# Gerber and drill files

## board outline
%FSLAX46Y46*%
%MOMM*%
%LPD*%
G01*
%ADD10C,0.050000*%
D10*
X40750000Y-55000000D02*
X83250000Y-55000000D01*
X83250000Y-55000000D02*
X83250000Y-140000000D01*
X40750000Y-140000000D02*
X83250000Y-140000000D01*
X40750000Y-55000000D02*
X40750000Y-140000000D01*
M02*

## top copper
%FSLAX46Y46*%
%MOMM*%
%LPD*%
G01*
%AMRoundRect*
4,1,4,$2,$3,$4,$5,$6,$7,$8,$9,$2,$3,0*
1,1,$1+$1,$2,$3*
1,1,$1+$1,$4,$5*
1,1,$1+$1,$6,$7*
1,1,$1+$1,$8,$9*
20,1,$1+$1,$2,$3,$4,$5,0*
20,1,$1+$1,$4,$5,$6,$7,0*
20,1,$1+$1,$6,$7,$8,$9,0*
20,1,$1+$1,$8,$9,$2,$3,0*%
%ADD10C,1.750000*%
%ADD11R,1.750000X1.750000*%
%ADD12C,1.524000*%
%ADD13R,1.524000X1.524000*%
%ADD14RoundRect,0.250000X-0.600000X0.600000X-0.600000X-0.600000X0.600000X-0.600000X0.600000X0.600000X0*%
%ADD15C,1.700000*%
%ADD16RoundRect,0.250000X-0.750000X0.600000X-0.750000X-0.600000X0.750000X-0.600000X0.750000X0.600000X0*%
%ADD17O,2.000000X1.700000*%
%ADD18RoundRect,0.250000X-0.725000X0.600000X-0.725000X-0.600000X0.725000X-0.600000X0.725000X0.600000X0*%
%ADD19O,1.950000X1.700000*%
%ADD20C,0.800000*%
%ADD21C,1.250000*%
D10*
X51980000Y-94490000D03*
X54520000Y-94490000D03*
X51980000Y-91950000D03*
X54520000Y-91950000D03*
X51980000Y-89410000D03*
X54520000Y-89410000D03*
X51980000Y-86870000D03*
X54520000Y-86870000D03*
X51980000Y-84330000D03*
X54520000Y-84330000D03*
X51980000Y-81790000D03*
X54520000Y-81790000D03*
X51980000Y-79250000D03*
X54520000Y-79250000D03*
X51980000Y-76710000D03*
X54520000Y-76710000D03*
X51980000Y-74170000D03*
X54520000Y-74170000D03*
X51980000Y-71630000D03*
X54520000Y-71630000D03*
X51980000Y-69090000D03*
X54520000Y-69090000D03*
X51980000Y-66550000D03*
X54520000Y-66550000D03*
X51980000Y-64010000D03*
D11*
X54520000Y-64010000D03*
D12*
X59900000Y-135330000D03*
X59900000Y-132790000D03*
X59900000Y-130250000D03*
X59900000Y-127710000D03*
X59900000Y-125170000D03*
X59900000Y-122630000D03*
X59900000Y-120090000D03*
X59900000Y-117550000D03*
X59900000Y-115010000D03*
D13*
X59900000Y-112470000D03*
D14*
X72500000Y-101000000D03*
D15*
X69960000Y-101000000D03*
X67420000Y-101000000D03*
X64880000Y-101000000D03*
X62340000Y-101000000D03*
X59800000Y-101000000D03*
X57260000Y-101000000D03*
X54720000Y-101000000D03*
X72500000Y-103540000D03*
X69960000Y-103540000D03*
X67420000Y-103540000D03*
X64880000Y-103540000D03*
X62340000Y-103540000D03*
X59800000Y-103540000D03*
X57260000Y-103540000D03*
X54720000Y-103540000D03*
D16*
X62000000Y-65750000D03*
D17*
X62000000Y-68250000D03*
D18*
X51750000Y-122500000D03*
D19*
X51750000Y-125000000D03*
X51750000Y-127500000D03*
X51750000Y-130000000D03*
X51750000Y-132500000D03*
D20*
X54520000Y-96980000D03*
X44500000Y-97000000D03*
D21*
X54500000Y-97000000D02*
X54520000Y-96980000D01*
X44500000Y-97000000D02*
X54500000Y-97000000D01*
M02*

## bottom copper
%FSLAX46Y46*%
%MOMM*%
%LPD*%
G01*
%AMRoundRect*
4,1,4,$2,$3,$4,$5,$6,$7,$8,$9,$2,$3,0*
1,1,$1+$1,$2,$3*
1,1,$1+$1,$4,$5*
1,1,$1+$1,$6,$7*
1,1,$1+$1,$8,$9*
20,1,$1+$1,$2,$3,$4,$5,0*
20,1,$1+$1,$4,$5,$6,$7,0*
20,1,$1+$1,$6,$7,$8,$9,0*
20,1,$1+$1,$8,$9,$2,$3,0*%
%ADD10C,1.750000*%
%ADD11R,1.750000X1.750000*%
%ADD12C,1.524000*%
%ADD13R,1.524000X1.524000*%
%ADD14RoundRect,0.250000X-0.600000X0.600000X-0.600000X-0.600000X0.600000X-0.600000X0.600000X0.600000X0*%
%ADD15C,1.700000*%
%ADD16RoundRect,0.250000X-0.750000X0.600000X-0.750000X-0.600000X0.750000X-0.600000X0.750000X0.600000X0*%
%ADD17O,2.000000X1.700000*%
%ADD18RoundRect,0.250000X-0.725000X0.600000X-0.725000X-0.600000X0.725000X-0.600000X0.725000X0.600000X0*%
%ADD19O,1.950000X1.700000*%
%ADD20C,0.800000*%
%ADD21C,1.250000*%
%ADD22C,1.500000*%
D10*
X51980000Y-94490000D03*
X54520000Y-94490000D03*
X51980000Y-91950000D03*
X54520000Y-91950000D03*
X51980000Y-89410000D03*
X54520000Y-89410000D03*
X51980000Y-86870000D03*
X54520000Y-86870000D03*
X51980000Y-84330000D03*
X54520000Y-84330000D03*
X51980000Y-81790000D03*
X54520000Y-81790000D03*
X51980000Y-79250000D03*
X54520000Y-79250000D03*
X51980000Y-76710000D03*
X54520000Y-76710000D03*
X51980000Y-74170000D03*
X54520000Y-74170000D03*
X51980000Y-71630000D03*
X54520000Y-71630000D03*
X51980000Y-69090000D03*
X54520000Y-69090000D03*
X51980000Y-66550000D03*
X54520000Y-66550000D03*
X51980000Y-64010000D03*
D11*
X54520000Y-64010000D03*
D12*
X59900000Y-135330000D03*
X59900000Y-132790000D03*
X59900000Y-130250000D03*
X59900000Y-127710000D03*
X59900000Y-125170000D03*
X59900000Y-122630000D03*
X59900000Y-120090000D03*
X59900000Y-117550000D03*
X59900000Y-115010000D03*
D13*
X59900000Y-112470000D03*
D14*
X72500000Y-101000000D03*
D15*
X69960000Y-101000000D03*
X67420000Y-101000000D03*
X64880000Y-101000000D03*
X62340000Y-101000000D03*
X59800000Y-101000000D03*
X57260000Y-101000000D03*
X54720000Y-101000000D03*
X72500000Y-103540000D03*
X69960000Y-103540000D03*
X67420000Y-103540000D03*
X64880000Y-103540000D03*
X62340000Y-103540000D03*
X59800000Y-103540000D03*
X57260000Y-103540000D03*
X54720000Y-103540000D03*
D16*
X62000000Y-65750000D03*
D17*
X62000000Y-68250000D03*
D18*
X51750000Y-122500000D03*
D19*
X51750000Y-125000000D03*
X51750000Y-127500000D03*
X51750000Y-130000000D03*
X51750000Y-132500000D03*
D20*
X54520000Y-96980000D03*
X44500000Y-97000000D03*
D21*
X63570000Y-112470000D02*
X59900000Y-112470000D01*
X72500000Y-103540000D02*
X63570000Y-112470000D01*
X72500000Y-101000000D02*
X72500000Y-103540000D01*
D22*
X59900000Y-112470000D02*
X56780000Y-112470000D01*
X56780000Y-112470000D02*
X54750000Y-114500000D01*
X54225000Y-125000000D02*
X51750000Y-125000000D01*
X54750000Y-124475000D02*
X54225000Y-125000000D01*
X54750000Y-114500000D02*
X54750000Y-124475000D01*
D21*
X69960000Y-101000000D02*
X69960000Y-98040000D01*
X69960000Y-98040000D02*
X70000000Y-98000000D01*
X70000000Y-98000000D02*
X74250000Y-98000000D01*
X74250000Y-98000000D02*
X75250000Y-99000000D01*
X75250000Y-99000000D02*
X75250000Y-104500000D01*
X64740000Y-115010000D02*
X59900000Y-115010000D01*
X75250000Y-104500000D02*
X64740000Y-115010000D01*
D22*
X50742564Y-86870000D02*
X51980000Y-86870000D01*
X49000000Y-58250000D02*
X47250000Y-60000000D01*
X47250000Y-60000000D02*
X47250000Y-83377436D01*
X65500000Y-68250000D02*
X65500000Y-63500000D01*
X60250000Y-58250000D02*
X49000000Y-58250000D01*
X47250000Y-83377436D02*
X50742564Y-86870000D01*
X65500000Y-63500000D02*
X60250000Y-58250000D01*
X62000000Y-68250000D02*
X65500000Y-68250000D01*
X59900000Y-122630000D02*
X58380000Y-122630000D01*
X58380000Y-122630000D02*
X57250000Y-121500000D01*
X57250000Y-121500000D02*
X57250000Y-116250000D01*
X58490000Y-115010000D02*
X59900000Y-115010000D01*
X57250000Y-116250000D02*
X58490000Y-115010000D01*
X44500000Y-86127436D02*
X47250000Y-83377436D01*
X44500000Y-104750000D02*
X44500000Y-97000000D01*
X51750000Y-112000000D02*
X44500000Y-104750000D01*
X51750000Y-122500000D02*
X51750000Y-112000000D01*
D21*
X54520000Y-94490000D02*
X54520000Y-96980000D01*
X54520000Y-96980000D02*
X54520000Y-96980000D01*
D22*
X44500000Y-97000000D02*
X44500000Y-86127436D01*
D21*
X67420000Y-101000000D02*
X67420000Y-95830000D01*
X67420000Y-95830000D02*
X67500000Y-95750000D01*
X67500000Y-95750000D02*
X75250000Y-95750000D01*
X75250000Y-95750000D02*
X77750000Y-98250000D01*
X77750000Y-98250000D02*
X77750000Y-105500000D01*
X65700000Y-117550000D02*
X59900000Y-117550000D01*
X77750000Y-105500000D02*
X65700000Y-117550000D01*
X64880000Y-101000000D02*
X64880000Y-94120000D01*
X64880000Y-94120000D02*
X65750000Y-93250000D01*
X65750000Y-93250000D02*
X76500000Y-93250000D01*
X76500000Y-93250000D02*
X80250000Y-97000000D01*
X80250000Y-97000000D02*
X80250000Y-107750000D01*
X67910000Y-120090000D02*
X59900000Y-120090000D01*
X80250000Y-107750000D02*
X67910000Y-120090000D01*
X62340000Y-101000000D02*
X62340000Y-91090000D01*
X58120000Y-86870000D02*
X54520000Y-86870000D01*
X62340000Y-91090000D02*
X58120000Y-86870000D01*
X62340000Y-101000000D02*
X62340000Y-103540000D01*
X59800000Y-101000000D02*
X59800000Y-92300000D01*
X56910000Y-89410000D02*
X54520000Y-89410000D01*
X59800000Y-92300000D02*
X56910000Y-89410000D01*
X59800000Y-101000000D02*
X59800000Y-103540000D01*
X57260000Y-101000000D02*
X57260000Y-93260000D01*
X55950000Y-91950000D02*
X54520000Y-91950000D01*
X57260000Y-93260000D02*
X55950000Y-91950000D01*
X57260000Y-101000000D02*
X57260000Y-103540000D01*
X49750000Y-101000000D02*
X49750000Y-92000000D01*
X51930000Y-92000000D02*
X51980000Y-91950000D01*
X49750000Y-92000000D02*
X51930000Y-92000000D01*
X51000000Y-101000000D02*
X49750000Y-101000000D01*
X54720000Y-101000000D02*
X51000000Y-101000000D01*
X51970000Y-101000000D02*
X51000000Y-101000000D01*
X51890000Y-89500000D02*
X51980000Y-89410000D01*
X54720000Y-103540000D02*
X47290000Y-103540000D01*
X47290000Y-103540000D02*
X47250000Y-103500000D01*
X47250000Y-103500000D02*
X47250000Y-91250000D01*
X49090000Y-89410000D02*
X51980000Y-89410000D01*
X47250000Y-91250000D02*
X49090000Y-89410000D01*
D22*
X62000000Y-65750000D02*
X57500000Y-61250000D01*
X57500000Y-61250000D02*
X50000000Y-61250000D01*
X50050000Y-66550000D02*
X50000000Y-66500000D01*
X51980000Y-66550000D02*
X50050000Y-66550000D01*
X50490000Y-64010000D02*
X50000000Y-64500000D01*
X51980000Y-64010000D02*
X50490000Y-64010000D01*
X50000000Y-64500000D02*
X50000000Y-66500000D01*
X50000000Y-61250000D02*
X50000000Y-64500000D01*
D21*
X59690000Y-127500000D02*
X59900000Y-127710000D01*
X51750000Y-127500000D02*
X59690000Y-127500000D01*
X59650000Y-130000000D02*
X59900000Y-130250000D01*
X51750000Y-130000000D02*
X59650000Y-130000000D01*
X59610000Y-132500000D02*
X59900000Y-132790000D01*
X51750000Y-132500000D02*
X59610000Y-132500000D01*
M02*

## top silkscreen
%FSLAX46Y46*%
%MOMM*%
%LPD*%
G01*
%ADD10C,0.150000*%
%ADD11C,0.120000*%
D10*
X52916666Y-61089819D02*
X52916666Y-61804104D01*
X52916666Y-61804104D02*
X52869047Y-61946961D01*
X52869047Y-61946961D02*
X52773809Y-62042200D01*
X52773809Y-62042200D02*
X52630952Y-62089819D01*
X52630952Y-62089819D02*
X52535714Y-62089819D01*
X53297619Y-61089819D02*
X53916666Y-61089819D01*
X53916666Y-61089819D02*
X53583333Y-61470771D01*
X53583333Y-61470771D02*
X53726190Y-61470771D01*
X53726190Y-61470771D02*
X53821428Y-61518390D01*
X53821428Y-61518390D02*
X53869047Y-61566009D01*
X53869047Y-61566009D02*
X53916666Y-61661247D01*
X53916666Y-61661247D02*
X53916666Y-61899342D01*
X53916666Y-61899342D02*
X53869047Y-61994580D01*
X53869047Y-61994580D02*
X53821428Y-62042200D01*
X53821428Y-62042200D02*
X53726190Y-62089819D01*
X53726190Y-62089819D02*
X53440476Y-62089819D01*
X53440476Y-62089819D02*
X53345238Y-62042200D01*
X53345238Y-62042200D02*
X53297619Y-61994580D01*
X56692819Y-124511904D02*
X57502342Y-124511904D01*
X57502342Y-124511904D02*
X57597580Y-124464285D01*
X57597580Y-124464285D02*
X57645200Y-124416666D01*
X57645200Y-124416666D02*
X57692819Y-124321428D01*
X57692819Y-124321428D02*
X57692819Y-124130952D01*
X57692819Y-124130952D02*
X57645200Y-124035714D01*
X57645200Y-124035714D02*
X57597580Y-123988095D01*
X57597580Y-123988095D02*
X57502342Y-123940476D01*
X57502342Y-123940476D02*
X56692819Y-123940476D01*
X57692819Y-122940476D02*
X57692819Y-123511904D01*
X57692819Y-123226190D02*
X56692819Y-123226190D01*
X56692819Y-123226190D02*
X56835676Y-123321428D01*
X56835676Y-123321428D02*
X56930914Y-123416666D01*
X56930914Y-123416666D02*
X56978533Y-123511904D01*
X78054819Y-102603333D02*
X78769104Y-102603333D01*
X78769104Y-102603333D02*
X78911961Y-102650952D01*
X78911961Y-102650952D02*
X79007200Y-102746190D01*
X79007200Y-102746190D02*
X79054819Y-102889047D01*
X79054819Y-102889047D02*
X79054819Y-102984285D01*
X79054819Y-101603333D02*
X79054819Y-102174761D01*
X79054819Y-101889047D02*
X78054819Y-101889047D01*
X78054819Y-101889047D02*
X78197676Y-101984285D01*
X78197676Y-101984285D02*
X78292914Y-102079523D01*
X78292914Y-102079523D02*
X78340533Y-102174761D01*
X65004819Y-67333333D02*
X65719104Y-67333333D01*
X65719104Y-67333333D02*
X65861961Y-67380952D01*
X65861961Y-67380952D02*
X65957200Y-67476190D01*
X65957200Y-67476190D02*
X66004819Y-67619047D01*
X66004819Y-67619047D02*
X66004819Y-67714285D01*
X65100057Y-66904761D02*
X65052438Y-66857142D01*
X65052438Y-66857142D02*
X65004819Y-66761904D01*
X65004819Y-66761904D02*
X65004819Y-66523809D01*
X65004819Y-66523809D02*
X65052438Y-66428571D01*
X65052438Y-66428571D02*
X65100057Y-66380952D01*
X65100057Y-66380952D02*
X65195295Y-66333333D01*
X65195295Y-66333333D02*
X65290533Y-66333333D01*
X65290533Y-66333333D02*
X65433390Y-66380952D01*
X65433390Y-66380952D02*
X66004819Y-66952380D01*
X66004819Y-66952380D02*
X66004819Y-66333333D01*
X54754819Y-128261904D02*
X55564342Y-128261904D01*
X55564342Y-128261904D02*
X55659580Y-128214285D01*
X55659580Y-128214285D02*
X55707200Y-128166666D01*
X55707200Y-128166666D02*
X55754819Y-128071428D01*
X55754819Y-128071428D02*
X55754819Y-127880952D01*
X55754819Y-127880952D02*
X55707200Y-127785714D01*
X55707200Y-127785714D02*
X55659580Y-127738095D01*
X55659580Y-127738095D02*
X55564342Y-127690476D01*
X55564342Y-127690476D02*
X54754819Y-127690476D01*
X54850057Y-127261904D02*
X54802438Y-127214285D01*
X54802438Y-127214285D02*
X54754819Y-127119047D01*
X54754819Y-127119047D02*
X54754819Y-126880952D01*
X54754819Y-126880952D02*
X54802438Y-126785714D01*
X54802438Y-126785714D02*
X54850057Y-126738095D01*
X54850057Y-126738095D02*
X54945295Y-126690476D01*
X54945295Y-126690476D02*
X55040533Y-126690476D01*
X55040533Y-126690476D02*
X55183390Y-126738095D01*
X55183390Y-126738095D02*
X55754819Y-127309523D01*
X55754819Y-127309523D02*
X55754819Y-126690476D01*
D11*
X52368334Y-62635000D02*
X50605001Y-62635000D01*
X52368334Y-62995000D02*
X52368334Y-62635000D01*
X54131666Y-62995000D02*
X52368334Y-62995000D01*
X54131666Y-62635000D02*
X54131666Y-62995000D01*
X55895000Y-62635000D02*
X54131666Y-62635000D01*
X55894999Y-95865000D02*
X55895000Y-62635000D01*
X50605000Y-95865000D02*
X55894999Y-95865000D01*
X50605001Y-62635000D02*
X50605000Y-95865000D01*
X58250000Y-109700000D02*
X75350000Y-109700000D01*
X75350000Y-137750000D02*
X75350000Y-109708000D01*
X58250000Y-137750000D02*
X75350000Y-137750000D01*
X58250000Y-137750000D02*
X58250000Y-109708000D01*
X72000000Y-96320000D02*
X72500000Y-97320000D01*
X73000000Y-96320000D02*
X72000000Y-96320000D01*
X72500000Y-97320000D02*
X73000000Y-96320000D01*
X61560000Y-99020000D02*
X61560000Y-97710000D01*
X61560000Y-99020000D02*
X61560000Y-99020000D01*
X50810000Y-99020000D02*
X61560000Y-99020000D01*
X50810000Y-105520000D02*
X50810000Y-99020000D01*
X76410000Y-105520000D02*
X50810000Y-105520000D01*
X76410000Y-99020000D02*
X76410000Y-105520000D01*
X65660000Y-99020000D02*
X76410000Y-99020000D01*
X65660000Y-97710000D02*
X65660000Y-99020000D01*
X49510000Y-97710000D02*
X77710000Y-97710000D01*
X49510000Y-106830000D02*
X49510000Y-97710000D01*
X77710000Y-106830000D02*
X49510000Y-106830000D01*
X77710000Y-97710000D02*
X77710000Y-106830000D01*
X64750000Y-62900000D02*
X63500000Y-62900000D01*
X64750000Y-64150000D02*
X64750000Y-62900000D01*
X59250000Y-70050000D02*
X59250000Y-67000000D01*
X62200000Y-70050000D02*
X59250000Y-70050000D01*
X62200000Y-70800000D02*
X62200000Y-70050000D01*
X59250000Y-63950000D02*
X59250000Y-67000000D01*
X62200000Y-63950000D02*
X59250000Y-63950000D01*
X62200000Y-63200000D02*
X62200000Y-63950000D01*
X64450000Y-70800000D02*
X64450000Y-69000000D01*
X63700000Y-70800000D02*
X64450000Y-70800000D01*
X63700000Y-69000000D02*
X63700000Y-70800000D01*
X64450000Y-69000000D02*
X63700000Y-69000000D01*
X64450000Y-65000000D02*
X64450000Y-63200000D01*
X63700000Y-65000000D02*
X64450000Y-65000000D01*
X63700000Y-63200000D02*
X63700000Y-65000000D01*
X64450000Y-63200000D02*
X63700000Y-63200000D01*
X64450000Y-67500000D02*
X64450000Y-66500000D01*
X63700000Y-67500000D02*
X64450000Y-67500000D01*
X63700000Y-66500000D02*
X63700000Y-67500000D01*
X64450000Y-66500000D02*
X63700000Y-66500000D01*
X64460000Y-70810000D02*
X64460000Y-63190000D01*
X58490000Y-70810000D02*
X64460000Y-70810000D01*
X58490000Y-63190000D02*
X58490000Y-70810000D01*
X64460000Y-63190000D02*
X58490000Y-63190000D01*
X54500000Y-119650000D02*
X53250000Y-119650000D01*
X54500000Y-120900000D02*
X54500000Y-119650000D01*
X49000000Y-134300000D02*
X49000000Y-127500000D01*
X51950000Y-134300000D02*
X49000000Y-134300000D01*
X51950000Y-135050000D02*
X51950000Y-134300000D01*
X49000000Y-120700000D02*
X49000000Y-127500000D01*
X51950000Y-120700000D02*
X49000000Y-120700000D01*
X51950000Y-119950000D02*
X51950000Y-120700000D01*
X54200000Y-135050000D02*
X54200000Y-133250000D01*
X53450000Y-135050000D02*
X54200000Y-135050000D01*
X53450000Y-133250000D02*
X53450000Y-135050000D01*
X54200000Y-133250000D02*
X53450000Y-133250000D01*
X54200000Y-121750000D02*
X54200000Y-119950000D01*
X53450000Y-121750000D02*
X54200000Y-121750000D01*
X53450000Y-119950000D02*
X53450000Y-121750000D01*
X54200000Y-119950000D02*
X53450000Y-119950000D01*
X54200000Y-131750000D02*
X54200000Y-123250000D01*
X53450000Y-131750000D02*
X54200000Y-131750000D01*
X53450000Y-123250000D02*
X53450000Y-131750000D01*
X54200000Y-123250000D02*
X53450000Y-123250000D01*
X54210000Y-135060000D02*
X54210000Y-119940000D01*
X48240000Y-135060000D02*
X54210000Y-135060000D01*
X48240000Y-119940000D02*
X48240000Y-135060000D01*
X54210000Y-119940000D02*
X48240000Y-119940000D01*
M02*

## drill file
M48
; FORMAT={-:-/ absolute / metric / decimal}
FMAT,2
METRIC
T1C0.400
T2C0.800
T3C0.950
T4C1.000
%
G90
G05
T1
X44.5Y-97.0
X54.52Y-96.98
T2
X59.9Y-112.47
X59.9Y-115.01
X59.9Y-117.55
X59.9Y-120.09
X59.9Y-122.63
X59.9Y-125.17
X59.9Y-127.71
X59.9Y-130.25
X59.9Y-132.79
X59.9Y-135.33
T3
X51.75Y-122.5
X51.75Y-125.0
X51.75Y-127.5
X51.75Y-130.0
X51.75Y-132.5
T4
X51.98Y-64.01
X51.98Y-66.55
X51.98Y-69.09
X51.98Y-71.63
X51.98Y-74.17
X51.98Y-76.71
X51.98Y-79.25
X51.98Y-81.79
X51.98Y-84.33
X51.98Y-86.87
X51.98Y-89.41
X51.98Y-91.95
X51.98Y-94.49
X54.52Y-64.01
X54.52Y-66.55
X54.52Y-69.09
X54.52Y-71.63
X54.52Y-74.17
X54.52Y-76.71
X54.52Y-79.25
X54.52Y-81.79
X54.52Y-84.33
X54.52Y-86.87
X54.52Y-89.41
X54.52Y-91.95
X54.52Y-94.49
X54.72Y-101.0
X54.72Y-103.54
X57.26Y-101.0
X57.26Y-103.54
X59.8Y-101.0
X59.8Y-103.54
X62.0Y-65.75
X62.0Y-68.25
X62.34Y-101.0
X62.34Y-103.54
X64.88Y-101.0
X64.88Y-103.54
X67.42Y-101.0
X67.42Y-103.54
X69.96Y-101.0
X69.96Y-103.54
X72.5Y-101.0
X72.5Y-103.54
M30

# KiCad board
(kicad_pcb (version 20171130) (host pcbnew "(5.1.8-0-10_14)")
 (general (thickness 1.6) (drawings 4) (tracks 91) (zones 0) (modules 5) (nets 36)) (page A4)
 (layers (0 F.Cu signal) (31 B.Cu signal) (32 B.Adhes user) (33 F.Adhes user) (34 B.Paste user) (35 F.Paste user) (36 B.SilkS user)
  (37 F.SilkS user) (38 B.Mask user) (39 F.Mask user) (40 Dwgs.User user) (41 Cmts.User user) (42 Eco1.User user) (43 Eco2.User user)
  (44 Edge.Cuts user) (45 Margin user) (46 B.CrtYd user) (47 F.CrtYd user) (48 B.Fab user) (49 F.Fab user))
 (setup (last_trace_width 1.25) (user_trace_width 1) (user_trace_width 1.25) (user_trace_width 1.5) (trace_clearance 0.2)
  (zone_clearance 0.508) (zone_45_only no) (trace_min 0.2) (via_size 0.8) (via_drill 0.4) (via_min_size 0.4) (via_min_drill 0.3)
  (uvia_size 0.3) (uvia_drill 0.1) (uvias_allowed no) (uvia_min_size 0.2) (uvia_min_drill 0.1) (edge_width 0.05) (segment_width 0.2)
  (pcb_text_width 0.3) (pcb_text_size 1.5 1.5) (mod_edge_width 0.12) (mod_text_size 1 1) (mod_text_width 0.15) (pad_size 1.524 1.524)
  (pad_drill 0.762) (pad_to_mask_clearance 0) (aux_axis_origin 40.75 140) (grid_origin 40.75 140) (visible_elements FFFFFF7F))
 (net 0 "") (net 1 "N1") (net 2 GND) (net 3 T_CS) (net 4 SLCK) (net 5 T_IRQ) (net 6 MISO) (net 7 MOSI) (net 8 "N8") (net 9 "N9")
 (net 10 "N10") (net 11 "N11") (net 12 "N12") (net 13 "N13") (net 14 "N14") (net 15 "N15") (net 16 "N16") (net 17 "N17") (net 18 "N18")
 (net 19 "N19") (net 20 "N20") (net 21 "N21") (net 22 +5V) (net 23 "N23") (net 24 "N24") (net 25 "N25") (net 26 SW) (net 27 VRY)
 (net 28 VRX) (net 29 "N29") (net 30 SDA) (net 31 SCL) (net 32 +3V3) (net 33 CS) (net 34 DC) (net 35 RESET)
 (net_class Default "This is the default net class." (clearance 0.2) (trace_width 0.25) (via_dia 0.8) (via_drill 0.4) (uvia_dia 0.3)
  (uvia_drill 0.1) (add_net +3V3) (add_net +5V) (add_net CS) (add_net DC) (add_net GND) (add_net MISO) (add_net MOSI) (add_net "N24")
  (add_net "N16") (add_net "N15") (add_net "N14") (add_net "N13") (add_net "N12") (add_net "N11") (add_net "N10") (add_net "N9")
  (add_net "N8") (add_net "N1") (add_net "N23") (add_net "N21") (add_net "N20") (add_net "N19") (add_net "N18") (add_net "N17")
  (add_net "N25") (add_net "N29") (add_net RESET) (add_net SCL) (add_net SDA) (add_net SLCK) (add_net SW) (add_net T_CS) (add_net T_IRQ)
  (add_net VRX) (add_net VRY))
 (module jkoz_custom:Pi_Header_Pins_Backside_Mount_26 (layer F.Cu) (at 53.25 79.25 270)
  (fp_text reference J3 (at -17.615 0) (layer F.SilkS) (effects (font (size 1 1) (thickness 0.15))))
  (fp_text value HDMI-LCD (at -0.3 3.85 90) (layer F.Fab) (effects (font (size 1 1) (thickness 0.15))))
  (fp_line (start -16.615 0.881666) (end -16.615 2.644999) (layer F.SilkS) (width 0.12))
  (fp_line (start -16.255 0.881666) (end -16.615 0.881666) (layer F.SilkS) (width 0.12))
  (fp_line (start -16.255 -0.881666) (end -16.255 0.881666) (layer F.SilkS) (width 0.12))
  (fp_line (start -16.615 -0.881666) (end -16.255 -0.881666) (layer F.SilkS) (width 0.12))
  (fp_line (start -16.615 -2.645) (end -16.615 -0.881666) (layer F.SilkS) (width 0.12))
  (fp_line (start 16.615 -2.644999) (end -16.615 -2.645) (layer F.SilkS) (width 0.12))
  (fp_line (start 16.615 2.645) (end 16.615 -2.644999) (layer F.SilkS) (width 0.12))
  (fp_line (start -16.615 2.644999) (end 16.615 2.645) (layer F.SilkS) (width 0.12))
  (pad 26 thru_hole circle (at 15.24 1.27 270) (size 1.75 1.75) (drill 1) (layers *.Cu *.Mask) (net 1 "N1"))
  (pad 25 thru_hole circle (at 15.24 -1.27 270) (size 1.75 1.75) (drill 1) (layers *.Cu *.Mask) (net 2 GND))
  (pad 24 thru_hole circle (at 12.7 1.27 270) (size 1.75 1.75) (drill 1) (layers *.Cu *.Mask) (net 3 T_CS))
  (pad 23 thru_hole circle (at 12.7 -1.27 270) (size 1.75 1.75) (drill 1) (layers *.Cu *.Mask) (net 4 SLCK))
  (pad 22 thru_hole circle (at 10.16 1.27 270) (size 1.75 1.75) (drill 1) (layers *.Cu *.Mask) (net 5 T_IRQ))
  (pad 21 thru_hole circle (at 10.16 -1.27 270) (size 1.75 1.75) (drill 1) (layers *.Cu *.Mask) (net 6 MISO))
  (pad 20 thru_hole circle (at 7.62 1.27 270) (size 1.75 1.75) (drill 1) (layers *.Cu *.Mask) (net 2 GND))
  (pad 19 thru_hole circle (at 7.62 -1.27 270) (size 1.75 1.75) (drill 1) (layers *.Cu *.Mask) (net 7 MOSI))
  (pad 18 thru_hole circle (at 5.08 1.27 270) (size 1.75 1.75) (drill 1) (layers *.Cu *.Mask) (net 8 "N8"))
  (pad 17 thru_hole circle (at 5.08 -1.27 270) (size 1.75 1.75) (drill 1) (layers *.Cu *.Mask) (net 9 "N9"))
  (pad 16 thru_hole circle (at 2.54 1.27 270) (size 1.75 1.75) (drill 1) (layers *.Cu *.Mask) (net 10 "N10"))
  (pad 15 thru_hole circle (at 2.54 -1.27 270) (size 1.75 1.75) (drill 1) (layers *.Cu *.Mask) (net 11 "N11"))
  (pad 14 thru_hole circle (at 0 1.27 270) (size 1.75 1.75) (drill 1) (layers *.Cu *.Mask) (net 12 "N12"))
  (pad 13 thru_hole circle (at 0 -1.27 270) (size 1.75 1.75) (drill 1) (layers *.Cu *.Mask) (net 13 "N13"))
  (pad 12 thru_hole circle (at -2.54 1.27 270) (size 1.75 1.75) (drill 1) (layers *.Cu *.Mask) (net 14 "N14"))
  (pad 11 thru_hole circle (at -2.54 -1.27 270) (size 1.75 1.75) (drill 1) (layers *.Cu *.Mask) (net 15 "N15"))
  (pad 10 thru_hole circle (at -5.08 1.27 270) (size 1.75 1.75) (drill 1) (layers *.Cu *.Mask) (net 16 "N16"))
  (pad 9 thru_hole circle (at -5.08 -1.27 270) (size 1.75 1.75) (drill 1) (layers *.Cu *.Mask) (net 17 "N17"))
  (pad 8 thru_hole circle (at -7.62 1.27 270) (size 1.75 1.75) (drill 1) (layers *.Cu *.Mask) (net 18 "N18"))
  (pad 7 thru_hole circle (at -7.62 -1.27 270) (size 1.75 1.75) (drill 1) (layers *.Cu *.Mask) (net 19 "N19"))
  (pad 6 thru_hole circle (at -10.16 1.27 270) (size 1.75 1.75) (drill 1) (layers *.Cu *.Mask) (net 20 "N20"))
  (pad 5 thru_hole circle (at -10.16 -1.27 270) (size 1.75 1.75) (drill 1) (layers *.Cu *.Mask) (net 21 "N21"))
  (pad 4 thru_hole circle (at -12.7 1.27 270) (size 1.75 1.75) (drill 1) (layers *.Cu *.Mask) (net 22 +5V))
  (pad 3 thru_hole circle (at -12.7 -1.27 270) (size 1.75 1.75) (drill 1) (layers *.Cu *.Mask) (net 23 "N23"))
  (pad 2 thru_hole circle (at -15.24 1.27 270) (size 1.75 1.75) (drill 1) (layers *.Cu *.Mask) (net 22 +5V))
  (pad 1 thru_hole rect (at -15.24 -1.27 270) (size 1.75 1.75) (drill 1) (layers *.Cu *.Mask) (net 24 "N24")))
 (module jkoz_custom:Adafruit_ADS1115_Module (layer F.Cu) (at 59.5 123.75 270)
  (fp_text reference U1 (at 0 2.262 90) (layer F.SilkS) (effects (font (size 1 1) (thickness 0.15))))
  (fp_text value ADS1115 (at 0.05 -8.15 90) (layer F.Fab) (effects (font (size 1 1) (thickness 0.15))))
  (fp_line (start -14.05 1.25) (end -14.05 -15.85) (layer F.SilkS) (width 0.12))
  (fp_line (start 14 -15.85) (end -14.042 -15.85) (layer F.SilkS) (width 0.12))
  (fp_line (start 14 1.25) (end 14 -15.85) (layer F.SilkS) (width 0.12))
  (fp_line (start 14 1.25) (end -14.042 1.25) (layer F.SilkS) (width 0.12))
  (pad 10 thru_hole circle (at 11.58 -0.4 270) (size 1.524 1.524) (drill 0.8) (layers *.Cu *.Mask) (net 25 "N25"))
  (pad 9 thru_hole circle (at 9.04 -0.4 270) (size 1.524 1.524) (drill 0.8) (layers *.Cu *.Mask) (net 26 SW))
  (pad 8 thru_hole circle (at 6.5 -0.4 270) (size 1.524 1.524) (drill 0.8) (layers *.Cu *.Mask) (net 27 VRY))
  (pad 7 thru_hole circle (at 3.96 -0.4 270) (size 1.524 1.524) (drill 0.8) (layers *.Cu *.Mask) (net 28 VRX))
  (pad 6 thru_hole circle (at 1.42 -0.4 270) (size 1.524 1.524) (drill 0.8) (layers *.Cu *.Mask) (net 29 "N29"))
  (pad 5 thru_hole circle (at -1.12 -0.4 270) (size 1.524 1.524) (drill 0.8) (layers *.Cu *.Mask) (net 2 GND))
  (pad 4 thru_hole circle (at -3.66 -0.4 270) (size 1.524 1.524) (drill 0.8) (layers *.Cu *.Mask) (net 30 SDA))
  (pad 3 thru_hole circle (at -6.2 -0.4 270) (size 1.524 1.524) (drill 0.8) (layers *.Cu *.Mask) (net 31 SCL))
  (pad 2 thru_hole circle (at -8.74 -0.4 270) (size 1.524 1.524) (drill 0.8) (layers *.Cu *.Mask) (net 2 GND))
  (pad 1 thru_hole rect (at -11.28 -0.4 270) (size 1.524 1.524) (drill 0.8) (layers *.Cu *.Mask) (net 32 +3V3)))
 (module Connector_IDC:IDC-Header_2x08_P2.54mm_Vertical (layer F.Cu) (at 72.5 101 270)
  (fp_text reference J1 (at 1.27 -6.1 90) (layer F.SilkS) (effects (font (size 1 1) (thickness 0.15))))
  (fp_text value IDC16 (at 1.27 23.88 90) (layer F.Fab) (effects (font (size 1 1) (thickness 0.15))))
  (fp_line (start -4.68 0.5) (end -3.68 0) (layer F.SilkS) (width 0.12))
  (fp_line (start -4.68 -0.5) (end -4.68 0.5) (layer F.SilkS) (width 0.12))
  (fp_line (start -3.68 0) (end -4.68 -0.5) (layer F.SilkS) (width 0.12))
  (fp_line (start -1.98 10.94) (end -3.29 10.94) (layer F.SilkS) (width 0.12))
  (fp_line (start -1.98 10.94) (end -1.98 10.94) (layer F.SilkS) (width 0.12))
  (fp_line (start -1.98 21.69) (end -1.98 10.94) (layer F.SilkS) (width 0.12))
  (fp_line (start 4.52 21.69) (end -1.98 21.69) (layer F.SilkS) (width 0.12))
  (fp_line (start 4.52 -3.91) (end 4.52 21.69) (layer F.SilkS) (width 0.12))
  (fp_line (start -1.98 -3.91) (end 4.52 -3.91) (layer F.SilkS) (width 0.12))
  (fp_line (start -1.98 6.84) (end -1.98 -3.91) (layer F.SilkS) (width 0.12))
  (fp_line (start -3.29 6.84) (end -1.98 6.84) (layer F.SilkS) (width 0.12))
  (fp_line (start -3.29 22.99) (end -3.29 -5.21) (layer F.SilkS) (width 0.12))
  (fp_line (start 5.83 22.99) (end -3.29 22.99) (layer F.SilkS) (width 0.12))
  (fp_line (start 5.83 -5.21) (end 5.83 22.99) (layer F.SilkS) (width 0.12))
  (fp_line (start -3.29 -5.21) (end 5.83 -5.21) (layer F.SilkS) (width 0.12))
  (pad 1 thru_hole roundrect (at 0 0 270) (size 1.7 1.7) (drill 1) (layers *.Cu *.Mask) (roundrect_rratio 0.1470588235294118) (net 32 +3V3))
  (pad 3 thru_hole circle (at 0 2.54 270) (size 1.7 1.7) (drill 1) (layers *.Cu *.Mask) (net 2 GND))
  (pad 5 thru_hole circle (at 0 5.08 270) (size 1.7 1.7) (drill 1) (layers *.Cu *.Mask) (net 31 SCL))
  (pad 7 thru_hole circle (at 0 7.62 270) (size 1.7 1.7) (drill 1) (layers *.Cu *.Mask) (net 30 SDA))
  (pad 9 thru_hole circle (at 0 10.16 270) (size 1.7 1.7) (drill 1) (layers *.Cu *.Mask) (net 7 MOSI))
  (pad 11 thru_hole circle (at 0 12.7 270) (size 1.7 1.7) (drill 1) (layers *.Cu *.Mask) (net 6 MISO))
  (pad 13 thru_hole circle (at 0 15.24 270) (size 1.7 1.7) (drill 1) (layers *.Cu *.Mask) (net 4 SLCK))
  (pad 15 thru_hole circle (at 0 17.78 270) (size 1.7 1.7) (drill 1) (layers *.Cu *.Mask) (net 3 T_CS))
  (pad 2 thru_hole circle (at 2.54 0 270) (size 1.7 1.7) (drill 1) (layers *.Cu *.Mask) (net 32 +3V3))
  (pad 4 thru_hole circle (at 2.54 2.54 270) (size 1.7 1.7) (drill 1) (layers *.Cu *.Mask) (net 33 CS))
  (pad 6 thru_hole circle (at 2.54 5.08 270) (size 1.7 1.7) (drill 1) (layers *.Cu *.Mask) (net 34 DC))
  (pad 8 thru_hole circle (at 2.54 7.62 270) (size 1.7 1.7) (drill 1) (layers *.Cu *.Mask) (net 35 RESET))
  (pad 10 thru_hole circle (at 2.54 10.16 270) (size 1.7 1.7) (drill 1) (layers *.Cu *.Mask) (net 7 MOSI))
  (pad 12 thru_hole circle (at 2.54 12.7 270) (size 1.7 1.7) (drill 1) (layers *.Cu *.Mask) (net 6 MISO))
  (pad 14 thru_hole circle (at 2.54 15.24 270) (size 1.7 1.7) (drill 1) (layers *.Cu *.Mask) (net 4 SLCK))
  (pad 16 thru_hole circle (at 2.54 17.78 270) (size 1.7 1.7) (drill 1) (layers *.Cu *.Mask) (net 5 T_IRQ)))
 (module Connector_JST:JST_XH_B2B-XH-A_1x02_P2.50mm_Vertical (layer F.Cu) (at 62 65.75 270)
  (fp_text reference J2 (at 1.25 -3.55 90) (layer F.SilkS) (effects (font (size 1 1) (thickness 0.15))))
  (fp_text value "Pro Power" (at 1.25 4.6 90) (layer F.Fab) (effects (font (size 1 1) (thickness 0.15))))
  (fp_line (start -2.85 -2.75) (end -2.85 -1.5) (layer F.SilkS) (width 0.12))
  (fp_line (start -1.6 -2.75) (end -2.85 -2.75) (layer F.SilkS) (width 0.12))
  (fp_line (start 4.3 2.75) (end 1.25 2.75) (layer F.SilkS) (width 0.12))
  (fp_line (start 4.3 -0.2) (end 4.3 2.75) (layer F.SilkS) (width 0.12))
  (fp_line (start 5.05 -0.2) (end 4.3 -0.2) (layer F.SilkS) (width 0.12))
  (fp_line (start -1.8 2.75) (end 1.25 2.75) (layer F.SilkS) (width 0.12))
  (fp_line (start -1.8 -0.2) (end -1.8 2.75) (layer F.SilkS) (width 0.12))
  (fp_line (start -2.55 -0.2) (end -1.8 -0.2) (layer F.SilkS) (width 0.12))
  (fp_line (start 5.05 -2.45) (end 3.25 -2.45) (layer F.SilkS) (width 0.12))
  (fp_line (start 5.05 -1.7) (end 5.05 -2.45) (layer F.SilkS) (width 0.12))
  (fp_line (start 3.25 -1.7) (end 5.05 -1.7) (layer F.SilkS) (width 0.12))
  (fp_line (start 3.25 -2.45) (end 3.25 -1.7) (layer F.SilkS) (width 0.12))
  (fp_line (start -0.75 -2.45) (end -2.55 -2.45) (layer F.SilkS) (width 0.12))
  (fp_line (start -0.75 -1.7) (end -0.75 -2.45) (layer F.SilkS) (width 0.12))
  (fp_line (start -2.55 -1.7) (end -0.75 -1.7) (layer F.SilkS) (width 0.12))
  (fp_line (start -2.55 -2.45) (end -2.55 -1.7) (layer F.SilkS) (width 0.12))
  (fp_line (start 1.75 -2.45) (end 0.75 -2.45) (layer F.SilkS) (width 0.12))
  (fp_line (start 1.75 -1.7) (end 1.75 -2.45) (layer F.SilkS) (width 0.12))
  (fp_line (start 0.75 -1.7) (end 1.75 -1.7) (layer F.SilkS) (width 0.12))
  (fp_line (start 0.75 -2.45) (end 0.75 -1.7) (layer F.SilkS) (width 0.12))
  (fp_line (start 5.06 -2.46) (end -2.56 -2.46) (layer F.SilkS) (width 0.12))
  (fp_line (start 5.06 3.51) (end 5.06 -2.46) (layer F.SilkS) (width 0.12))
  (fp_line (start -2.56 3.51) (end 5.06 3.51) (layer F.SilkS) (width 0.12))
  (fp_line (start -2.56 -2.46) (end -2.56 3.51) (layer F.SilkS) (width 0.12))
  (pad 1 thru_hole roundrect (at 0 0 270) (size 1.7 2) (drill 1) (layers *.Cu *.Mask) (roundrect_rratio 0.1470588235294118) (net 22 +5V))
  (pad 2 thru_hole oval (at 2.5 0 270) (size 1.7 2) (drill 1) (layers *.Cu *.Mask) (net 2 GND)))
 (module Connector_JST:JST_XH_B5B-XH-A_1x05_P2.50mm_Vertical (layer F.Cu) (at 51.75 122.5 270)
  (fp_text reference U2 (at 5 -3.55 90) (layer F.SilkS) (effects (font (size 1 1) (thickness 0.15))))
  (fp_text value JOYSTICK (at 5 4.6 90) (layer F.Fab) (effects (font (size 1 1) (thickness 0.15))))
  (fp_line (start -2.85 -2.75) (end -2.85 -1.5) (layer F.SilkS) (width 0.12))
  (fp_line (start -1.6 -2.75) (end -2.85 -2.75) (layer F.SilkS) (width 0.12))
  (fp_line (start 11.8 2.75) (end 5 2.75) (layer F.SilkS) (width 0.12))
  (fp_line (start 11.8 -0.2) (end 11.8 2.75) (layer F.SilkS) (width 0.12))
  (fp_line (start 12.55 -0.2) (end 11.8 -0.2) (layer F.SilkS) (width 0.12))
  (fp_line (start -1.8 2.75) (end 5 2.75) (layer F.SilkS) (width 0.12))
  (fp_line (start -1.8 -0.2) (end -1.8 2.75) (layer F.SilkS) (width 0.12))
  (fp_line (start -2.55 -0.2) (end -1.8 -0.2) (layer F.SilkS) (width 0.12))
  (fp_line (start 12.55 -2.45) (end 10.75 -2.45) (layer F.SilkS) (width 0.12))
  (fp_line (start 12.55 -1.7) (end 12.55 -2.45) (layer F.SilkS) (width 0.12))
  (fp_line (start 10.75 -1.7) (end 12.55 -1.7) (layer F.SilkS) (width 0.12))
  (fp_line (start 10.75 -2.45) (end 10.75 -1.7) (layer F.SilkS) (width 0.12))
  (fp_line (start -0.75 -2.45) (end -2.55 -2.45) (layer F.SilkS) (width 0.12))
  (fp_line (start -0.75 -1.7) (end -0.75 -2.45) (layer F.SilkS) (width 0.12))
  (fp_line (start -2.55 -1.7) (end -0.75 -1.7) (layer F.SilkS) (width 0.12))
  (fp_line (start -2.55 -2.45) (end -2.55 -1.7) (layer F.SilkS) (width 0.12))
  (fp_line (start 9.25 -2.45) (end 0.75 -2.45) (layer F.SilkS) (width 0.12))
  (fp_line (start 9.25 -1.7) (end 9.25 -2.45) (layer F.SilkS) (width 0.12))
  (fp_line (start 0.75 -1.7) (end 9.25 -1.7) (layer F.SilkS) (width 0.12))
  (fp_line (start 0.75 -2.45) (end 0.75 -1.7) (layer F.SilkS) (width 0.12))
  (fp_line (start 12.56 -2.46) (end -2.56 -2.46) (layer F.SilkS) (width 0.12))
  (fp_line (start 12.56 3.51) (end 12.56 -2.46) (layer F.SilkS) (width 0.12))
  (fp_line (start -2.56 3.51) (end 12.56 3.51) (layer F.SilkS) (width 0.12))
  (fp_line (start -2.56 -2.46) (end -2.56 3.51) (layer F.SilkS) (width 0.12))
  (pad 1 thru_hole roundrect (at 0 0 270) (size 1.7 1.95) (drill 0.95) (layers *.Cu *.Mask) (roundrect_rratio 0.1470588235294118)
   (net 2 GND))
  (pad 2 thru_hole oval (at 2.5 0 270) (size 1.7 1.95) (drill 0.95) (layers *.Cu *.Mask) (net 32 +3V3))
  (pad 3 thru_hole oval (at 5 0 270) (size 1.7 1.95) (drill 0.95) (layers *.Cu *.Mask) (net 28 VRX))
  (pad 4 thru_hole oval (at 7.5 0 270) (size 1.7 1.95) (drill 0.95) (layers *.Cu *.Mask) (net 27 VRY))
  (pad 5 thru_hole oval (at 10 0 270) (size 1.7 1.95) (drill 0.95) (layers *.Cu *.Mask) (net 26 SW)))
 (gr_line (start 40.75 55) (end 83.25 55) (layer Edge.Cuts) (width 0.05))
 (gr_line (start 83.25 55) (end 83.25 140) (layer Edge.Cuts) (width 0.05))
 (gr_line (start 40.75 140) (end 83.25 140) (layer Edge.Cuts) (width 0.05))
 (gr_line (start 40.75 55) (end 40.75 140) (layer Edge.Cuts) (width 0.05))
 (segment (start 63.57 112.47) (end 59.9 112.47) (width 1.25) (layer B.Cu) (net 32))
 (segment (start 72.5 103.54) (end 63.57 112.47) (width 1.25) (layer B.Cu) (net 32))
 (segment (start 72.5 101) (end 72.5 103.54) (width 1.25) (layer B.Cu) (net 32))
 (segment (start 59.9 112.47) (end 56.78 112.47) (width 1.5) (layer B.Cu) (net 32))
 (segment (start 56.78 112.47) (end 54.75 114.5) (width 1.5) (layer B.Cu) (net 32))
 (segment (start 54.225 125) (end 51.75 125) (width 1.5) (layer B.Cu) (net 32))
 (segment (start 54.75 124.475) (end 54.225 125) (width 1.5) (layer B.Cu) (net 32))
 (segment (start 54.75 114.5) (end 54.75 124.475) (width 1.5) (layer B.Cu) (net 32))
 (segment (start 69.96 101) (end 69.96 98.04) (width 1.25) (layer B.Cu) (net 2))
 (segment (start 69.96 98.04) (end 70 98) (width 1.25) (layer B.Cu) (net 2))
 (segment (start 70 98) (end 74.25 98) (width 1.25) (layer B.Cu) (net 2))
 (segment (start 74.25 98) (end 75.25 99) (width 1.25) (layer B.Cu) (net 2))
 (segment (start 75.25 99) (end 75.25 104.5) (width 1.25) (layer B.Cu) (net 2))
 (segment (start 64.74 115.01) (end 59.9 115.01) (width 1.25) (layer B.Cu) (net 2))
 (segment (start 75.25 104.5) (end 64.74 115.01) (width 1.25) (layer B.Cu) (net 2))
 (segment (start 50.742564 86.87) (end 51.98 86.87) (width 1.5) (layer B.Cu) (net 2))
 (segment (start 49 58.25) (end 47.25 60) (width 1.5) (layer B.Cu) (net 2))
 (segment (start 47.25 60) (end 47.25 83.377436) (width 1.5) (layer B.Cu) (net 2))
 (segment (start 65.5 68.25) (end 65.5 63.5) (width 1.5) (layer B.Cu) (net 2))
 (segment (start 60.25 58.25) (end 49 58.25) (width 1.5) (layer B.Cu) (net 2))
 (segment (start 47.25 83.377436) (end 50.742564 86.87) (width 1.5) (layer B.Cu) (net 2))
 (segment (start 65.5 63.5) (end 60.25 58.25) (width 1.5) (layer B.Cu) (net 2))
 (segment (start 62 68.25) (end 65.5 68.25) (width 1.5) (layer B.Cu) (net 2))
 (segment (start 59.9 122.63) (end 58.38 122.63) (width 1.5) (layer B.Cu) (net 2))
 (segment (start 58.38 122.63) (end 57.25 121.5) (width 1.5) (layer B.Cu) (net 2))
 (segment (start 57.25 121.5) (end 57.25 116.25) (width 1.5) (layer B.Cu) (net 2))
 (segment (start 58.49 115.01) (end 59.9 115.01) (width 1.5) (layer B.Cu) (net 2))
 (segment (start 57.25 116.25) (end 58.49 115.01) (width 1.5) (layer B.Cu) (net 2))
 (segment (start 44.5 86.127436) (end 47.25 83.377436) (width 1.5) (layer B.Cu) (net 2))
 (segment (start 44.5 104.75) (end 44.5 97) (width 1.5) (layer B.Cu) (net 2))
 (segment (start 51.75 112) (end 44.5 104.75) (width 1.5) (layer B.Cu) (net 2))
 (segment (start 51.75 122.5) (end 51.75 112) (width 1.5) (layer B.Cu) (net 2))
 (segment (start 54.52 94.49) (end 54.52 96.98) (width 1.25) (layer B.Cu) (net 2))
 (segment (start 54.52 96.98) (end 54.52 96.98) (width 1.25) (layer B.Cu) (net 2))
 (via (at 54.52 96.98) (size 0.8) (drill 0.4) (layers F.Cu B.Cu) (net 2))
 (segment (start 44.5 97) (end 44.5 86.127436) (width 1.5) (layer B.Cu) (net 2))
 (via (at 44.5 97) (size 0.8) (drill 0.4) (layers F.Cu B.Cu) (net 2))
 (segment (start 54.5 97) (end 54.52 96.98) (width 1.25) (layer F.Cu) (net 2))
 (segment (start 44.5 97) (end 54.5 97) (width 1.25) (layer F.Cu) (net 2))
 (segment (start 67.42 101) (end 67.42 95.83) (width 1.25) (layer B.Cu) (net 31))
 (segment (start 67.42 95.83) (end 67.5 95.75) (width 1.25) (layer B.Cu) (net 31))
 (segment (start 67.5 95.75) (end 75.25 95.75) (width 1.25) (layer B.Cu) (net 31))
 (segment (start 75.25 95.75) (end 77.75 98.25) (width 1.25) (layer B.Cu) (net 31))
 (segment (start 77.75 98.25) (end 77.75 105.5) (width 1.25) (layer B.Cu) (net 31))
 (segment (start 65.7 117.55) (end 59.9 117.55) (width 1.25) (layer B.Cu) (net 31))
 (segment (start 77.75 105.5) (end 65.7 117.55) (width 1.25) (layer B.Cu) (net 31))
 (segment (start 64.88 101) (end 64.88 94.12) (width 1.25) (layer B.Cu) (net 30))
 (segment (start 64.88 94.12) (end 65.75 93.25) (width 1.25) (layer B.Cu) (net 30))
 (segment (start 65.75 93.25) (end 76.5 93.25) (width 1.25) (layer B.Cu) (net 30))
 (segment (start 76.5 93.25) (end 80.25 97) (width 1.25) (layer B.Cu) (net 30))
 (segment (start 80.25 97) (end 80.25 107.75) (width 1.25) (layer B.Cu) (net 30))
 (segment (start 67.91 120.09) (end 59.9 120.09) (width 1.25) (layer B.Cu) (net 30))
 (segment (start 80.25 107.75) (end 67.91 120.09) (width 1.25) (layer B.Cu) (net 30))
 (segment (start 62.34 101) (end 62.34 91.09) (width 1.25) (layer B.Cu) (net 7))
 (segment (start 58.12 86.87) (end 54.52 86.87) (width 1.25) (layer B.Cu) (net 7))
 (segment (start 62.34 91.09) (end 58.12 86.87) (width 1.25) (layer B.Cu) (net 7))
 (segment (start 62.34 101) (end 62.34 103.54) (width 1.25) (layer B.Cu) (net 7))
 (segment (start 59.8 101) (end 59.8 92.3) (width 1.25) (layer B.Cu) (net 6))
 (segment (start 56.91 89.41) (end 54.52 89.41) (width 1.25) (layer B.Cu) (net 6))
 (segment (start 59.8 92.3) (end 56.91 89.41) (width 1.25) (layer B.Cu) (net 6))
 (segment (start 59.8 101) (end 59.8 103.54) (width 1.25) (layer B.Cu) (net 6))
 (segment (start 57.26 101) (end 57.26 93.26) (width 1.25) (layer B.Cu) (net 4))
 (segment (start 55.95 91.95) (end 54.52 91.95) (width 1.25) (layer B.Cu) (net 4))
 (segment (start 57.26 93.26) (end 55.95 91.95) (width 1.25) (layer B.Cu) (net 4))
 (segment (start 57.26 101) (end 57.26 103.54) (width 1.25) (layer B.Cu) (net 4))
 (segment (start 49.75 101) (end 49.75 92) (width 1.25) (layer B.Cu) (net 3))
 (segment (start 51.93 92) (end 51.98 91.95) (width 1.25) (layer B.Cu) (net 3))
 (segment (start 49.75 92) (end 51.93 92) (width 1.25) (layer B.Cu) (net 3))
 (segment (start 51 101) (end 49.75 101) (width 1.25) (layer B.Cu) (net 3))
 (segment (start 54.72 101) (end 51 101) (width 1.25) (layer B.Cu) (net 3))
 (segment (start 51.97 101) (end 51 101) (width 1.25) (layer B.Cu) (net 3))
 (segment (start 51.89 89.5) (end 51.98 89.41) (width 1.25) (layer B.Cu) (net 5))
 (segment (start 54.72 103.54) (end 47.29 103.54) (width 1.25) (layer B.Cu) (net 5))
 (segment (start 47.29 103.54) (end 47.25 103.5) (width 1.25) (layer B.Cu) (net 5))
 (segment (start 47.25 103.5) (end 47.25 91.25) (width 1.25) (layer B.Cu) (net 5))
 (segment (start 49.09 89.41) (end 51.98 89.41) (width 1.25) (layer B.Cu) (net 5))
 (segment (start 47.25 91.25) (end 49.09 89.41) (width 1.25) (layer B.Cu) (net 5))
 (segment (start 62 65.75) (end 57.5 61.25) (width 1.5) (layer B.Cu) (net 22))
 (segment (start 57.5 61.25) (end 50 61.25) (width 1.5) (layer B.Cu) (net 22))
 (segment (start 50.05 66.55) (end 50 66.5) (width 1.5) (layer B.Cu) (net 22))
 (segment (start 51.98 66.55) (end 50.05 66.55) (width 1.5) (layer B.Cu) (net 22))
 (segment (start 50.49 64.01) (end 50 64.5) (width 1.5) (layer B.Cu) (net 22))
 (segment (start 51.98 64.01) (end 50.49 64.01) (width 1.5) (layer B.Cu) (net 22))
 (segment (start 50 64.5) (end 50 66.5) (width 1.5) (layer B.Cu) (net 22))
 (segment (start 50 61.25) (end 50 64.5) (width 1.5) (layer B.Cu) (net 22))
 (segment (start 59.69 127.5) (end 59.9 127.71) (width 1.25) (layer B.Cu) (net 28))
 (segment (start 51.75 127.5) (end 59.69 127.5) (width 1.25) (layer B.Cu) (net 28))
 (segment (start 59.65 130) (end 59.9 130.25) (width 1.25) (layer B.Cu) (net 27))
 (segment (start 51.75 130) (end 59.65 130) (width 1.25) (layer B.Cu) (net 27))
 (segment (start 59.61 132.5) (end 59.9 132.79) (width 1.25) (layer B.Cu) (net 26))
 (segment (start 51.75 132.5) (end 59.61 132.5) (width 1.25) (layer B.Cu) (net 26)))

